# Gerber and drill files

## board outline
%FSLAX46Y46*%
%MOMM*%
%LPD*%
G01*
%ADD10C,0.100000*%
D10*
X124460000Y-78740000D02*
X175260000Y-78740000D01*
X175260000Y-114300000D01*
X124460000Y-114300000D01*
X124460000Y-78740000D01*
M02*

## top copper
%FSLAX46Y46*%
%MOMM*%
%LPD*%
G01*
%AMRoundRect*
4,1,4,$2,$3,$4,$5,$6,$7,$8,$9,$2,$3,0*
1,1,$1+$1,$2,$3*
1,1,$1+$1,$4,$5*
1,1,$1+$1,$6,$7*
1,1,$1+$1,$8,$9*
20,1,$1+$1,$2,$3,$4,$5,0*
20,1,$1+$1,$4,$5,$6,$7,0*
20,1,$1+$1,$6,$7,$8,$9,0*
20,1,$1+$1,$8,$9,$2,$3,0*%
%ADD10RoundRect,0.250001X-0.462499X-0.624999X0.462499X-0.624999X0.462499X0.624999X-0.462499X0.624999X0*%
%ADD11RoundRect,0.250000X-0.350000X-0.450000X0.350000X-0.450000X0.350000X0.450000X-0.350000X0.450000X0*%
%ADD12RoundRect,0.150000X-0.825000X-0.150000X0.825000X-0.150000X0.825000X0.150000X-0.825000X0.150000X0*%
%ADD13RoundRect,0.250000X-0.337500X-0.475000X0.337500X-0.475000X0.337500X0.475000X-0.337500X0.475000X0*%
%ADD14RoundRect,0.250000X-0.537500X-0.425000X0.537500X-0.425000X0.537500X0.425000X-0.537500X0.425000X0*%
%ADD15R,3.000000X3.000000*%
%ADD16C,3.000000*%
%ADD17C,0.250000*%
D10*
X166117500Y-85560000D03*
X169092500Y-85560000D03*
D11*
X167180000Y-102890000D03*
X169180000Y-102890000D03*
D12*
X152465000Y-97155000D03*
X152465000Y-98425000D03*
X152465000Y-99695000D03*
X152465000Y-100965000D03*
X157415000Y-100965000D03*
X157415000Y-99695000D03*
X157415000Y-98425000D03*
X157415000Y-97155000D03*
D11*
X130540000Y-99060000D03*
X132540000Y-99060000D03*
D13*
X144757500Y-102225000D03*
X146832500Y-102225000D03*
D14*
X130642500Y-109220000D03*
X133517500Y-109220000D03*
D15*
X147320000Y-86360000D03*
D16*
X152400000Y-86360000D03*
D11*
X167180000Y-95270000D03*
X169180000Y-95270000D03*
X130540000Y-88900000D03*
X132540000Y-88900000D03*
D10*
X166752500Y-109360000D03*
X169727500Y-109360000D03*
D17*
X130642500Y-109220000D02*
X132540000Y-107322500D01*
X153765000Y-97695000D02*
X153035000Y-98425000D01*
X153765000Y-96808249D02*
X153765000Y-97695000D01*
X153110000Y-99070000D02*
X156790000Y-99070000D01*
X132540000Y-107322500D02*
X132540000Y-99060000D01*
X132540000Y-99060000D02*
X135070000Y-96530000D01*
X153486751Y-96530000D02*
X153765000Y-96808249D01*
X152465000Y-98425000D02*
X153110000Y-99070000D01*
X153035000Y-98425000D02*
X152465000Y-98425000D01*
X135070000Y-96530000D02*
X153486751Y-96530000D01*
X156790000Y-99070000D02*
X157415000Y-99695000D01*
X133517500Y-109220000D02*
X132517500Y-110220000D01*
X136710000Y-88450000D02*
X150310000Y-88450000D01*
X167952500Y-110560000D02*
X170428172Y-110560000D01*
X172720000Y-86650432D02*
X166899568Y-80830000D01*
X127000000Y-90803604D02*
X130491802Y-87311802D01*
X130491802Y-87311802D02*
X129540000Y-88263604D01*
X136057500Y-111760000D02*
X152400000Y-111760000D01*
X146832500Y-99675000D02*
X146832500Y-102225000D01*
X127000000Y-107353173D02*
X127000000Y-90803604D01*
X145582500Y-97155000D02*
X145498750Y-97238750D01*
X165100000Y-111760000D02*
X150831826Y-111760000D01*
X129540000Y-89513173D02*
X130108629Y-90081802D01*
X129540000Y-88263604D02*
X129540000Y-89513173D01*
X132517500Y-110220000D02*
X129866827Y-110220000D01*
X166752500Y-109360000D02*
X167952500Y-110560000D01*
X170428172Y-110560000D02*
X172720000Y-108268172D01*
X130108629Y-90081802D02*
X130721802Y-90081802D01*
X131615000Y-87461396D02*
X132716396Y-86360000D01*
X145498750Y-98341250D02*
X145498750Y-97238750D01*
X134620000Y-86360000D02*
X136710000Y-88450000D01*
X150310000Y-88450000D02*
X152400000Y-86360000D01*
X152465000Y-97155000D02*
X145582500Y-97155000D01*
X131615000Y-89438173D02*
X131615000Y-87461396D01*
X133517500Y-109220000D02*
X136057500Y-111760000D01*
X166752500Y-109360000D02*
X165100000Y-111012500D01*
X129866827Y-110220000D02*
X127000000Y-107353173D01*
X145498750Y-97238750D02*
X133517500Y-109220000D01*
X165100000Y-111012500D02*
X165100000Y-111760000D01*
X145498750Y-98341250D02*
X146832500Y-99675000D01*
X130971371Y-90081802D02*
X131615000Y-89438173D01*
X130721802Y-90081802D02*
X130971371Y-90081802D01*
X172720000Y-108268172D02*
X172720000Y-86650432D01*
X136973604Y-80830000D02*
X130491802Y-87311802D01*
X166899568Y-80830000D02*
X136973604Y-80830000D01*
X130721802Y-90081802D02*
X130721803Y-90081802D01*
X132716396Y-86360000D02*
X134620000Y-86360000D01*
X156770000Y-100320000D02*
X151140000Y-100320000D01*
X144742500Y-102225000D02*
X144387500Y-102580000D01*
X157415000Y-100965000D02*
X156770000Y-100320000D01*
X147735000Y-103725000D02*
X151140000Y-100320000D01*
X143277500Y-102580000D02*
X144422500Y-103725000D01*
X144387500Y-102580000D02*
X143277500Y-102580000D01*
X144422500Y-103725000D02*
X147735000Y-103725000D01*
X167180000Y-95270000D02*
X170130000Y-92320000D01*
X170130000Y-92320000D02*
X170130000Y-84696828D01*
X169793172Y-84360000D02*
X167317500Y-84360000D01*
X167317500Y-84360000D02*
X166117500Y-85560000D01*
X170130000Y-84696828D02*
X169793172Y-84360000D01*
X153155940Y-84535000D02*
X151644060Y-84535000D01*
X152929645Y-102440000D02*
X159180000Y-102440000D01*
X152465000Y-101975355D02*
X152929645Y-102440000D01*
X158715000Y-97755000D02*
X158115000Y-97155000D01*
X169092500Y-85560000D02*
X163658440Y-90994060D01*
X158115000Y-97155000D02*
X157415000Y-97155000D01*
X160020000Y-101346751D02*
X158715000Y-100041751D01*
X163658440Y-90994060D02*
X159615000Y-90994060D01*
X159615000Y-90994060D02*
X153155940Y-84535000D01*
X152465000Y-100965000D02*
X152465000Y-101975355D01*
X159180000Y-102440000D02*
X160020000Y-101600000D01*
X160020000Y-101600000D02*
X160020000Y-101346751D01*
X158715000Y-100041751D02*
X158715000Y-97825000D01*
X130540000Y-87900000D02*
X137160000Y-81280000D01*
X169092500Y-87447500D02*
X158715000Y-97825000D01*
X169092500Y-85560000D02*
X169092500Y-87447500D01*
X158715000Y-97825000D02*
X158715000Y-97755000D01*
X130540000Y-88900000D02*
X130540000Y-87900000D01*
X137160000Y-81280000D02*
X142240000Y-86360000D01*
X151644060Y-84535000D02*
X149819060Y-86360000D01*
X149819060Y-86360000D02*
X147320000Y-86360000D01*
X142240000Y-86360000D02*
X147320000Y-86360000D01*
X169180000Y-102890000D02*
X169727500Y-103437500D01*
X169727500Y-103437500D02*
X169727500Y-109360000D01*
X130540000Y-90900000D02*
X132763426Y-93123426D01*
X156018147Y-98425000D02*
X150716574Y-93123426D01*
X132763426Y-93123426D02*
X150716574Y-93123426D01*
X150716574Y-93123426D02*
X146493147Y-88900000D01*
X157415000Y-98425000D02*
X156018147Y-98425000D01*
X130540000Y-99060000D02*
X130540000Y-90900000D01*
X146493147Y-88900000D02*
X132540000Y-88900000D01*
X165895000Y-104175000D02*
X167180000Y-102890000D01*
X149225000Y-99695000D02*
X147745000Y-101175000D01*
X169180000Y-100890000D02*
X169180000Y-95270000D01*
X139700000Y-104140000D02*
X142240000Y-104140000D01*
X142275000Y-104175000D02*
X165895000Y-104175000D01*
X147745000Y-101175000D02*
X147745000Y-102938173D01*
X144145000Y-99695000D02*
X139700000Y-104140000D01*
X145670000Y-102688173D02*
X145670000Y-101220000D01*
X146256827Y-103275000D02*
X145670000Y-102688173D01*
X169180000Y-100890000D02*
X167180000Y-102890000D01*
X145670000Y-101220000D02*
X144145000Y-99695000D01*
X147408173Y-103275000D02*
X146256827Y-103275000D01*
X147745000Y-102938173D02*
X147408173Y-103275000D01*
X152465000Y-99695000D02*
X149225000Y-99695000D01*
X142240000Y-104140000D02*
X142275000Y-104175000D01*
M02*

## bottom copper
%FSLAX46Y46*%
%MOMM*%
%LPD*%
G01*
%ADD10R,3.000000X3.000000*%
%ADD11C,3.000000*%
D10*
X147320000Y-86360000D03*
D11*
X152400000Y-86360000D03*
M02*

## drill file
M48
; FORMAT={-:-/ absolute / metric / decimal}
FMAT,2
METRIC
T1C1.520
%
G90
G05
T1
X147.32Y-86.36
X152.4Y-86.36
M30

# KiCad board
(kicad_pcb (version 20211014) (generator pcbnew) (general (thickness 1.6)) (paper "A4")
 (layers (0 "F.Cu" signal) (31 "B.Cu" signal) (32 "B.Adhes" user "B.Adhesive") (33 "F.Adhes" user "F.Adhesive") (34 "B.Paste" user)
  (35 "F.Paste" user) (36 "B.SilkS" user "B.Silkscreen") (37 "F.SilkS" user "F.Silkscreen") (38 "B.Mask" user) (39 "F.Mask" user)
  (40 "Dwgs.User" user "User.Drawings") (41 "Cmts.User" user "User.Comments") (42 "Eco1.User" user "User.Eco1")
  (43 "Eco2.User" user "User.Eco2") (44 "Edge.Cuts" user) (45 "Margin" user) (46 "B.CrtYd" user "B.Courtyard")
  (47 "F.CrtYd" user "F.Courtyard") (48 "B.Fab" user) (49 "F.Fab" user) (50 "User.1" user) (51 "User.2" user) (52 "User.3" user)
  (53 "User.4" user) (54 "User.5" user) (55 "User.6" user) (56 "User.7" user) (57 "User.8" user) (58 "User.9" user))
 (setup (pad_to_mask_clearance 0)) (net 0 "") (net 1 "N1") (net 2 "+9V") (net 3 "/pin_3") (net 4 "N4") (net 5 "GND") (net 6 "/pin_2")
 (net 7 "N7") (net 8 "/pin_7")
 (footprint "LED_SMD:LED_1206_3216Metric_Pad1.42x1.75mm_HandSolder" (layer "F.Cu") (at 167.605 85.56)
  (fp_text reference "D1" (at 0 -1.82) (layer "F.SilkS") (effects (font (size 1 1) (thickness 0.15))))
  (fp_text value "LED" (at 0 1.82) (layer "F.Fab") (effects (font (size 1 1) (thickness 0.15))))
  (pad "1" smd roundrect (at -1.4875 0) (size 1.425 1.75) (layers "F.Cu" "F.Paste" "F.Mask") (roundrect_rratio 0.175439) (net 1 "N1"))
  (pad "2" smd roundrect (at 1.4875 0) (size 1.425 1.75) (layers "F.Cu" "F.Paste" "F.Mask") (roundrect_rratio 0.175439) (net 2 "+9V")))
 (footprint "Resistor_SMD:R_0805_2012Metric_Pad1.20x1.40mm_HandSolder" (layer "F.Cu") (at 168.18 102.89)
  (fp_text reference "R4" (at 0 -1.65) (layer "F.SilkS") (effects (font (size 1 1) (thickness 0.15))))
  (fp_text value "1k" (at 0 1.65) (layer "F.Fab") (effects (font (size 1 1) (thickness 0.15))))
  (pad "1" smd roundrect (at -1 0) (size 1.2 1.4) (layers "F.Cu" "F.Paste" "F.Mask") (roundrect_rratio 0.208333) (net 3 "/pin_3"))
  (pad "2" smd roundrect (at 1 0) (size 1.2 1.4) (layers "F.Cu" "F.Paste" "F.Mask") (roundrect_rratio 0.208333) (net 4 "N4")))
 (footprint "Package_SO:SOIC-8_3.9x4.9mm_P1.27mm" (layer "F.Cu") (at 154.94 99.06)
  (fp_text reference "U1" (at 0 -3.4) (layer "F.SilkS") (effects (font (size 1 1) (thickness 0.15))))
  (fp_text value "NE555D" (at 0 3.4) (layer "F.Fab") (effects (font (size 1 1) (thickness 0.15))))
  (pad "1" smd roundrect (at -2.475 -1.905) (size 1.95 0.6) (layers "F.Cu" "F.Paste" "F.Mask") (roundrect_rratio 0.25) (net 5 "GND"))
  (pad "2" smd roundrect (at -2.475 -0.635) (size 1.95 0.6) (layers "F.Cu" "F.Paste" "F.Mask") (roundrect_rratio 0.25) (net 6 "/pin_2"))
  (pad "3" smd roundrect (at -2.475 0.635) (size 1.95 0.6) (layers "F.Cu" "F.Paste" "F.Mask") (roundrect_rratio 0.25) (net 3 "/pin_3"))
  (pad "4" smd roundrect (at -2.475 1.905) (size 1.95 0.6) (layers "F.Cu" "F.Paste" "F.Mask") (roundrect_rratio 0.25) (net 2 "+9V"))
  (pad "5" smd roundrect (at 2.475 1.905) (size 1.95 0.6) (layers "F.Cu" "F.Paste" "F.Mask") (roundrect_rratio 0.25) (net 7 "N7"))
  (pad "6" smd roundrect (at 2.475 0.635) (size 1.95 0.6) (layers "F.Cu" "F.Paste" "F.Mask") (roundrect_rratio 0.25) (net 6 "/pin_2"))
  (pad "7" smd roundrect (at 2.475 -0.635) (size 1.95 0.6) (layers "F.Cu" "F.Paste" "F.Mask") (roundrect_rratio 0.25) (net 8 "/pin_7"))
  (pad "8" smd roundrect (at 2.475 -1.905) (size 1.95 0.6) (layers "F.Cu" "F.Paste" "F.Mask") (roundrect_rratio 0.25) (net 2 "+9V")))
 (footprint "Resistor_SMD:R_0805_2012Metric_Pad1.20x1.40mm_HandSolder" (layer "F.Cu") (at 131.54 99.06)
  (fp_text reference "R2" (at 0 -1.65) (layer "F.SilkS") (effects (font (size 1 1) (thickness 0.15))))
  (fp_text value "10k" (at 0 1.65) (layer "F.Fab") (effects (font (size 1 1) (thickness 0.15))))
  (pad "1" smd roundrect (at -1 0) (size 1.2 1.4) (layers "F.Cu" "F.Paste" "F.Mask") (roundrect_rratio 0.208333) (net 8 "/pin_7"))
  (pad "2" smd roundrect (at 1 0) (size 1.2 1.4) (layers "F.Cu" "F.Paste" "F.Mask") (roundrect_rratio 0.208333) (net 6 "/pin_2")))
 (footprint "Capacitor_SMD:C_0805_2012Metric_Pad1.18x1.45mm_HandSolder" (layer "F.Cu") (at 145.795 102.225)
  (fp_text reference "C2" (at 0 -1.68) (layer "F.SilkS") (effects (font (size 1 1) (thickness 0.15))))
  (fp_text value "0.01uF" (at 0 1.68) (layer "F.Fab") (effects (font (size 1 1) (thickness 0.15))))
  (pad "1" smd roundrect (at -1.0375 0) (size 1.175 1.45) (layers "F.Cu" "F.Paste" "F.Mask") (roundrect_rratio 0.212766) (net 7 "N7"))
  (pad "2" smd roundrect (at 1.0375 0) (size 1.175 1.45) (layers "F.Cu" "F.Paste" "F.Mask") (roundrect_rratio 0.212766) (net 5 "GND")))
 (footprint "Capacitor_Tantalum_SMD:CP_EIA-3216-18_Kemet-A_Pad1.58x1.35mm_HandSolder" (layer "F.Cu") (at 132.08 109.22)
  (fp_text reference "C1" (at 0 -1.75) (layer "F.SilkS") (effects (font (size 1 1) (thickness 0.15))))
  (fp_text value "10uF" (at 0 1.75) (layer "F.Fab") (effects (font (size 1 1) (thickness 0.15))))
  (pad "1" smd roundrect (at -1.4375 0) (size 1.575 1.35) (layers "F.Cu" "F.Paste" "F.Mask") (roundrect_rratio 0.185185) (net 6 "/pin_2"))
  (pad "2" smd roundrect (at 1.4375 0) (size 1.575 1.35) (layers "F.Cu" "F.Paste" "F.Mask") (roundrect_rratio 0.185185) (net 5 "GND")))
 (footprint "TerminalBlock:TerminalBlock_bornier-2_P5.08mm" (layer "F.Cu") (at 147.32 86.36)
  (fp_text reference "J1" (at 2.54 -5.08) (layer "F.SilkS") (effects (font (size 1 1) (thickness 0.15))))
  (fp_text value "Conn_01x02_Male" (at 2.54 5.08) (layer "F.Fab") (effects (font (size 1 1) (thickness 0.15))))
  (pad "1" thru_hole rect (at 0 0) (size 3 3) (drill 1.52) (layers *.Cu *.Mask) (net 2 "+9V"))
  (pad "2" thru_hole circle (at 5.08 0) (size 3 3) (drill 1.52) (layers *.Cu *.Mask) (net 5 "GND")))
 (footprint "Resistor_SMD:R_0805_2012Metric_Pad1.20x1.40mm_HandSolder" (layer "F.Cu") (at 168.18 95.27)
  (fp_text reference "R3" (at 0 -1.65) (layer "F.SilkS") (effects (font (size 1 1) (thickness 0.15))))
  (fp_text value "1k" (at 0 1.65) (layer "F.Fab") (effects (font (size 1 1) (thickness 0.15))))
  (pad "1" smd roundrect (at -1 0) (size 1.2 1.4) (layers "F.Cu" "F.Paste" "F.Mask") (roundrect_rratio 0.208333) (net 1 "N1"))
  (pad "2" smd roundrect (at 1 0) (size 1.2 1.4) (layers "F.Cu" "F.Paste" "F.Mask") (roundrect_rratio 0.208333) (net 3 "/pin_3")))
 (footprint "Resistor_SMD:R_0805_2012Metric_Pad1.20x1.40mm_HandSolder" (layer "F.Cu") (at 131.54 88.9)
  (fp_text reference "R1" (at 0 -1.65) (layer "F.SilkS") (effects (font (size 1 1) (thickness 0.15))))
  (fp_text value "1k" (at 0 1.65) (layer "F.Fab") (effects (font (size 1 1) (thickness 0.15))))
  (pad "1" smd roundrect (at -1 0) (size 1.2 1.4) (layers "F.Cu" "F.Paste" "F.Mask") (roundrect_rratio 0.208333) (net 2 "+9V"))
  (pad "2" smd roundrect (at 1 0) (size 1.2 1.4) (layers "F.Cu" "F.Paste" "F.Mask") (roundrect_rratio 0.208333) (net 8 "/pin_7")))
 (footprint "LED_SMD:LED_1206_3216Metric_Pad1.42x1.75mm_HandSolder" (layer "F.Cu") (at 168.24 109.36)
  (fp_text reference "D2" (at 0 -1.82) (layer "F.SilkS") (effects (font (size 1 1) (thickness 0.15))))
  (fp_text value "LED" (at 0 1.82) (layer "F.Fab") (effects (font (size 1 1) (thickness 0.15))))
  (pad "1" smd roundrect (at -1.4875 0) (size 1.425 1.75) (layers "F.Cu" "F.Paste" "F.Mask") (roundrect_rratio 0.175439) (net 5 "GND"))
  (pad "2" smd roundrect (at 1.4875 0) (size 1.425 1.75) (layers "F.Cu" "F.Paste" "F.Mask") (roundrect_rratio 0.175439) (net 4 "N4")))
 (gr_rect (start 124.46 78.74) (end 175.26 114.3) (layer "Edge.Cuts") (width 0.1) (fill none))
 (segment (start 130.6425 109.22) (end 132.54 107.3225) (width 0.25) (layer "F.Cu") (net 6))
 (segment (start 153.765 97.695) (end 153.035 98.425) (width 0.25) (layer "F.Cu") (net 6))
 (segment (start 153.765 96.808249) (end 153.765 97.695) (width 0.25) (layer "F.Cu") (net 6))
 (segment (start 153.11 99.07) (end 156.79 99.07) (width 0.25) (layer "F.Cu") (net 6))
 (segment (start 132.54 107.3225) (end 132.54 99.06) (width 0.25) (layer "F.Cu") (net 6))
 (segment (start 132.54 99.06) (end 135.07 96.53) (width 0.25) (layer "F.Cu") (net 6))
 (segment (start 153.486751 96.53) (end 153.765 96.808249) (width 0.25) (layer "F.Cu") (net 6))
 (segment (start 152.465 98.425) (end 153.11 99.07) (width 0.25) (layer "F.Cu") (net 6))
 (segment (start 153.035 98.425) (end 152.465 98.425) (width 0.25) (layer "F.Cu") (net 6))
 (segment (start 135.07 96.53) (end 153.486751 96.53) (width 0.25) (layer "F.Cu") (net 6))
 (segment (start 156.79 99.07) (end 157.415 99.695) (width 0.25) (layer "F.Cu") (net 6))
 (segment (start 133.5175 109.22) (end 132.5175 110.22) (width 0.25) (layer "F.Cu") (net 5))
 (segment (start 136.71 88.45) (end 150.31 88.45) (width 0.25) (layer "F.Cu") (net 5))
 (segment (start 167.9525 110.56) (end 170.428172 110.56) (width 0.25) (layer "F.Cu") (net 5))
 (segment (start 172.72 86.650432) (end 166.899568 80.83) (width 0.25) (layer "F.Cu") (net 5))
 (segment (start 127 90.803604) (end 130.491802 87.311802) (width 0.25) (layer "F.Cu") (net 5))
 (segment (start 130.491802 87.311802) (end 129.54 88.263604) (width 0.25) (layer "F.Cu") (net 5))
 (segment (start 136.0575 111.76) (end 152.4 111.76) (width 0.25) (layer "F.Cu") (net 5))
 (segment (start 146.8325 99.675) (end 146.8325 102.225) (width 0.25) (layer "F.Cu") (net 5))
 (segment (start 127 107.353173) (end 127 90.803604) (width 0.25) (layer "F.Cu") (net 5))
 (segment (start 145.5825 97.155) (end 145.49875 97.23875) (width 0.25) (layer "F.Cu") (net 5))
 (segment (start 165.1 111.76) (end 150.831826 111.76) (width 0.25) (layer "F.Cu") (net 5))
 (segment (start 129.54 89.513173) (end 130.108629 90.081802) (width 0.25) (layer "F.Cu") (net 5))
 (segment (start 129.54 88.263604) (end 129.54 89.513173) (width 0.25) (layer "F.Cu") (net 5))
 (segment (start 132.5175 110.22) (end 129.866827 110.22) (width 0.25) (layer "F.Cu") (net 5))
 (segment (start 166.7525 109.36) (end 167.9525 110.56) (width 0.25) (layer "F.Cu") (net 5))
 (segment (start 170.428172 110.56) (end 172.72 108.268172) (width 0.25) (layer "F.Cu") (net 5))
 (segment (start 130.108629 90.081802) (end 130.721802 90.081802) (width 0.25) (layer "F.Cu") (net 5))
 (segment (start 131.615 87.461396) (end 132.716396 86.36) (width 0.25) (layer "F.Cu") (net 5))
 (segment (start 145.49875 98.34125) (end 145.49875 97.23875) (width 0.25) (layer "F.Cu") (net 5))
 (segment (start 134.62 86.36) (end 136.71 88.45) (width 0.25) (layer "F.Cu") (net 5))
 (segment (start 150.31 88.45) (end 152.4 86.36) (width 0.25) (layer "F.Cu") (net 5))
 (segment (start 152.465 97.155) (end 145.5825 97.155) (width 0.25) (layer "F.Cu") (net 5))
 (segment (start 131.615 89.438173) (end 131.615 87.461396) (width 0.25) (layer "F.Cu") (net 5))
 (segment (start 133.5175 109.22) (end 136.0575 111.76) (width 0.25) (layer "F.Cu") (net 5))
 (segment (start 166.7525 109.36) (end 165.1 111.0125) (width 0.25) (layer "F.Cu") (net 5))
 (segment (start 129.866827 110.22) (end 127 107.353173) (width 0.25) (layer "F.Cu") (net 5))
 (segment (start 145.49875 97.23875) (end 133.5175 109.22) (width 0.25) (layer "F.Cu") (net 5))
 (segment (start 165.1 111.0125) (end 165.1 111.76) (width 0.25) (layer "F.Cu") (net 5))
 (segment (start 145.49875 98.34125) (end 146.8325 99.675) (width 0.25) (layer "F.Cu") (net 5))
 (segment (start 130.971371 90.081802) (end 131.615 89.438173) (width 0.25) (layer "F.Cu") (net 5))
 (segment (start 130.721802 90.081802) (end 130.971371 90.081802) (width 0.25) (layer "F.Cu") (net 5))
 (segment (start 172.72 108.268172) (end 172.72 86.650432) (width 0.25) (layer "F.Cu") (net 5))
 (segment (start 136.973604 80.83) (end 130.491802 87.311802) (width 0.25) (layer "F.Cu") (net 5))
 (segment (start 166.899568 80.83) (end 136.973604 80.83) (width 0.25) (layer "F.Cu") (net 5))
 (segment (start 130.721802 90.081802) (end 130.721803 90.081802) (width 0.25) (layer "F.Cu") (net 5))
 (segment (start 132.716396 86.36) (end 134.62 86.36) (width 0.25) (layer "F.Cu") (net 5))
 (segment (start 156.77 100.32) (end 151.14 100.32) (width 0.25) (layer "F.Cu") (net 7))
 (segment (start 144.7425 102.225) (end 144.3875 102.58) (width 0.25) (layer "F.Cu") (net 7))
 (segment (start 157.415 100.965) (end 156.77 100.32) (width 0.25) (layer "F.Cu") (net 7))
 (segment (start 147.735 103.725) (end 151.14 100.32) (width 0.25) (layer "F.Cu") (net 7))
 (segment (start 143.2775 102.58) (end 144.4225 103.725) (width 0.25) (layer "F.Cu") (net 7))
 (segment (start 144.3875 102.58) (end 143.2775 102.58) (width 0.25) (layer "F.Cu") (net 7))
 (segment (start 144.4225 103.725) (end 147.735 103.725) (width 0.25) (layer "F.Cu") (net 7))
 (segment (start 167.18 95.27) (end 170.13 92.32) (width 0.25) (layer "F.Cu") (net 1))
 (segment (start 170.13 92.32) (end 170.13 84.696828) (width 0.25) (layer "F.Cu") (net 1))
 (segment (start 169.793172 84.36) (end 167.3175 84.36) (width 0.25) (layer "F.Cu") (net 1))
 (segment (start 167.3175 84.36) (end 166.1175 85.56) (width 0.25) (layer "F.Cu") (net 1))
 (segment (start 170.13 84.696828) (end 169.793172 84.36) (width 0.25) (layer "F.Cu") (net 1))
 (segment (start 153.15594 84.535) (end 151.64406 84.535) (width 0.25) (layer "F.Cu") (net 2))
 (segment (start 152.929645 102.44) (end 159.18 102.44) (width 0.25) (layer "F.Cu") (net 2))
 (segment (start 152.465 101.975355) (end 152.929645 102.44) (width 0.25) (layer "F.Cu") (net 2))
 (segment (start 158.715 97.755) (end 158.115 97.155) (width 0.25) (layer "F.Cu") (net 2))
 (segment (start 169.0925 85.56) (end 163.65844 90.99406) (width 0.25) (layer "F.Cu") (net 2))
 (segment (start 158.115 97.155) (end 157.415 97.155) (width 0.25) (layer "F.Cu") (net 2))
 (segment (start 160.02 101.346751) (end 158.715 100.041751) (width 0.25) (layer "F.Cu") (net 2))
 (segment (start 163.65844 90.99406) (end 159.615 90.99406) (width 0.25) (layer "F.Cu") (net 2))
 (segment (start 159.615 90.99406) (end 153.15594 84.535) (width 0.25) (layer "F.Cu") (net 2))
 (segment (start 152.465 100.965) (end 152.465 101.975355) (width 0.25) (layer "F.Cu") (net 2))
 (segment (start 159.18 102.44) (end 160.02 101.6) (width 0.25) (layer "F.Cu") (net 2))
 (segment (start 160.02 101.6) (end 160.02 101.346751) (width 0.25) (layer "F.Cu") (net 2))
 (segment (start 158.715 100.041751) (end 158.715 97.825) (width 0.25) (layer "F.Cu") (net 2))
 (segment (start 130.54 87.9) (end 137.16 81.28) (width 0.25) (layer "F.Cu") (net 2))
 (segment (start 169.0925 87.4475) (end 158.715 97.825) (width 0.25) (layer "F.Cu") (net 2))
 (segment (start 169.0925 85.56) (end 169.0925 87.4475) (width 0.25) (layer "F.Cu") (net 2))
 (segment (start 158.715 97.825) (end 158.715 97.755) (width 0.25) (layer "F.Cu") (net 2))
 (segment (start 130.54 88.9) (end 130.54 87.9) (width 0.25) (layer "F.Cu") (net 2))
 (segment (start 137.16 81.28) (end 142.24 86.36) (width 0.25) (layer "F.Cu") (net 2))
 (segment (start 151.64406 84.535) (end 149.81906 86.36) (width 0.25) (layer "F.Cu") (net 2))
 (segment (start 149.81906 86.36) (end 147.32 86.36) (width 0.25) (layer "F.Cu") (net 2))
 (segment (start 142.24 86.36) (end 147.32 86.36) (width 0.25) (layer "F.Cu") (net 2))
 (segment (start 169.18 102.89) (end 169.7275 103.4375) (width 0.25) (layer "F.Cu") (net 4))
 (segment (start 169.7275 103.4375) (end 169.7275 109.36) (width 0.25) (layer "F.Cu") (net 4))
 (segment (start 130.54 90.9) (end 132.763426 93.123426) (width 0.25) (layer "F.Cu") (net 8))
 (segment (start 156.018147 98.425) (end 150.716574 93.123426) (width 0.25) (layer "F.Cu") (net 8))
 (segment (start 132.763426 93.123426) (end 150.716574 93.123426) (width 0.25) (layer "F.Cu") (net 8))
 (segment (start 150.716574 93.123426) (end 146.493147 88.9) (width 0.25) (layer "F.Cu") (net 8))
 (segment (start 157.415 98.425) (end 156.018147 98.425) (width 0.25) (layer "F.Cu") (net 8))
 (segment (start 130.54 99.06) (end 130.54 90.9) (width 0.25) (layer "F.Cu") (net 8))
 (segment (start 146.493147 88.9) (end 132.54 88.9) (width 0.25) (layer "F.Cu") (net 8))
 (segment (start 165.895 104.175) (end 167.18 102.89) (width 0.25) (layer "F.Cu") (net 3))
 (segment (start 149.225 99.695) (end 147.745 101.175) (width 0.25) (layer "F.Cu") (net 3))
 (segment (start 169.18 100.89) (end 169.18 95.27) (width 0.25) (layer "F.Cu") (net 3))
 (segment (start 139.7 104.14) (end 142.24 104.14) (width 0.25) (layer "F.Cu") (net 3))
 (segment (start 142.275 104.175) (end 165.895 104.175) (width 0.25) (layer "F.Cu") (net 3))
 (segment (start 147.745 101.175) (end 147.745 102.938173) (width 0.25) (layer "F.Cu") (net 3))
 (segment (start 144.145 99.695) (end 139.7 104.14) (width 0.25) (layer "F.Cu") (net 3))
 (segment (start 145.67 102.688173) (end 145.67 101.22) (width 0.25) (layer "F.Cu") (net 3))
 (segment (start 146.256827 103.275) (end 145.67 102.688173) (width 0.25) (layer "F.Cu") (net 3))
 (segment (start 169.18 100.89) (end 167.18 102.89) (width 0.25) (layer "F.Cu") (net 3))
 (segment (start 145.67 101.22) (end 144.145 99.695) (width 0.25) (layer "F.Cu") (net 3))
 (segment (start 147.408173 103.275) (end 146.256827 103.275) (width 0.25) (layer "F.Cu") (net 3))
 (segment (start 147.745 102.938173) (end 147.408173 103.275) (width 0.25) (layer "F.Cu") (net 3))
 (segment (start 152.465 99.695) (end 149.225 99.695) (width 0.25) (layer "F.Cu") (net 3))
 (segment (start 142.24 104.14) (end 142.275 104.175) (width 0.25) (layer "F.Cu") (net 3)))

